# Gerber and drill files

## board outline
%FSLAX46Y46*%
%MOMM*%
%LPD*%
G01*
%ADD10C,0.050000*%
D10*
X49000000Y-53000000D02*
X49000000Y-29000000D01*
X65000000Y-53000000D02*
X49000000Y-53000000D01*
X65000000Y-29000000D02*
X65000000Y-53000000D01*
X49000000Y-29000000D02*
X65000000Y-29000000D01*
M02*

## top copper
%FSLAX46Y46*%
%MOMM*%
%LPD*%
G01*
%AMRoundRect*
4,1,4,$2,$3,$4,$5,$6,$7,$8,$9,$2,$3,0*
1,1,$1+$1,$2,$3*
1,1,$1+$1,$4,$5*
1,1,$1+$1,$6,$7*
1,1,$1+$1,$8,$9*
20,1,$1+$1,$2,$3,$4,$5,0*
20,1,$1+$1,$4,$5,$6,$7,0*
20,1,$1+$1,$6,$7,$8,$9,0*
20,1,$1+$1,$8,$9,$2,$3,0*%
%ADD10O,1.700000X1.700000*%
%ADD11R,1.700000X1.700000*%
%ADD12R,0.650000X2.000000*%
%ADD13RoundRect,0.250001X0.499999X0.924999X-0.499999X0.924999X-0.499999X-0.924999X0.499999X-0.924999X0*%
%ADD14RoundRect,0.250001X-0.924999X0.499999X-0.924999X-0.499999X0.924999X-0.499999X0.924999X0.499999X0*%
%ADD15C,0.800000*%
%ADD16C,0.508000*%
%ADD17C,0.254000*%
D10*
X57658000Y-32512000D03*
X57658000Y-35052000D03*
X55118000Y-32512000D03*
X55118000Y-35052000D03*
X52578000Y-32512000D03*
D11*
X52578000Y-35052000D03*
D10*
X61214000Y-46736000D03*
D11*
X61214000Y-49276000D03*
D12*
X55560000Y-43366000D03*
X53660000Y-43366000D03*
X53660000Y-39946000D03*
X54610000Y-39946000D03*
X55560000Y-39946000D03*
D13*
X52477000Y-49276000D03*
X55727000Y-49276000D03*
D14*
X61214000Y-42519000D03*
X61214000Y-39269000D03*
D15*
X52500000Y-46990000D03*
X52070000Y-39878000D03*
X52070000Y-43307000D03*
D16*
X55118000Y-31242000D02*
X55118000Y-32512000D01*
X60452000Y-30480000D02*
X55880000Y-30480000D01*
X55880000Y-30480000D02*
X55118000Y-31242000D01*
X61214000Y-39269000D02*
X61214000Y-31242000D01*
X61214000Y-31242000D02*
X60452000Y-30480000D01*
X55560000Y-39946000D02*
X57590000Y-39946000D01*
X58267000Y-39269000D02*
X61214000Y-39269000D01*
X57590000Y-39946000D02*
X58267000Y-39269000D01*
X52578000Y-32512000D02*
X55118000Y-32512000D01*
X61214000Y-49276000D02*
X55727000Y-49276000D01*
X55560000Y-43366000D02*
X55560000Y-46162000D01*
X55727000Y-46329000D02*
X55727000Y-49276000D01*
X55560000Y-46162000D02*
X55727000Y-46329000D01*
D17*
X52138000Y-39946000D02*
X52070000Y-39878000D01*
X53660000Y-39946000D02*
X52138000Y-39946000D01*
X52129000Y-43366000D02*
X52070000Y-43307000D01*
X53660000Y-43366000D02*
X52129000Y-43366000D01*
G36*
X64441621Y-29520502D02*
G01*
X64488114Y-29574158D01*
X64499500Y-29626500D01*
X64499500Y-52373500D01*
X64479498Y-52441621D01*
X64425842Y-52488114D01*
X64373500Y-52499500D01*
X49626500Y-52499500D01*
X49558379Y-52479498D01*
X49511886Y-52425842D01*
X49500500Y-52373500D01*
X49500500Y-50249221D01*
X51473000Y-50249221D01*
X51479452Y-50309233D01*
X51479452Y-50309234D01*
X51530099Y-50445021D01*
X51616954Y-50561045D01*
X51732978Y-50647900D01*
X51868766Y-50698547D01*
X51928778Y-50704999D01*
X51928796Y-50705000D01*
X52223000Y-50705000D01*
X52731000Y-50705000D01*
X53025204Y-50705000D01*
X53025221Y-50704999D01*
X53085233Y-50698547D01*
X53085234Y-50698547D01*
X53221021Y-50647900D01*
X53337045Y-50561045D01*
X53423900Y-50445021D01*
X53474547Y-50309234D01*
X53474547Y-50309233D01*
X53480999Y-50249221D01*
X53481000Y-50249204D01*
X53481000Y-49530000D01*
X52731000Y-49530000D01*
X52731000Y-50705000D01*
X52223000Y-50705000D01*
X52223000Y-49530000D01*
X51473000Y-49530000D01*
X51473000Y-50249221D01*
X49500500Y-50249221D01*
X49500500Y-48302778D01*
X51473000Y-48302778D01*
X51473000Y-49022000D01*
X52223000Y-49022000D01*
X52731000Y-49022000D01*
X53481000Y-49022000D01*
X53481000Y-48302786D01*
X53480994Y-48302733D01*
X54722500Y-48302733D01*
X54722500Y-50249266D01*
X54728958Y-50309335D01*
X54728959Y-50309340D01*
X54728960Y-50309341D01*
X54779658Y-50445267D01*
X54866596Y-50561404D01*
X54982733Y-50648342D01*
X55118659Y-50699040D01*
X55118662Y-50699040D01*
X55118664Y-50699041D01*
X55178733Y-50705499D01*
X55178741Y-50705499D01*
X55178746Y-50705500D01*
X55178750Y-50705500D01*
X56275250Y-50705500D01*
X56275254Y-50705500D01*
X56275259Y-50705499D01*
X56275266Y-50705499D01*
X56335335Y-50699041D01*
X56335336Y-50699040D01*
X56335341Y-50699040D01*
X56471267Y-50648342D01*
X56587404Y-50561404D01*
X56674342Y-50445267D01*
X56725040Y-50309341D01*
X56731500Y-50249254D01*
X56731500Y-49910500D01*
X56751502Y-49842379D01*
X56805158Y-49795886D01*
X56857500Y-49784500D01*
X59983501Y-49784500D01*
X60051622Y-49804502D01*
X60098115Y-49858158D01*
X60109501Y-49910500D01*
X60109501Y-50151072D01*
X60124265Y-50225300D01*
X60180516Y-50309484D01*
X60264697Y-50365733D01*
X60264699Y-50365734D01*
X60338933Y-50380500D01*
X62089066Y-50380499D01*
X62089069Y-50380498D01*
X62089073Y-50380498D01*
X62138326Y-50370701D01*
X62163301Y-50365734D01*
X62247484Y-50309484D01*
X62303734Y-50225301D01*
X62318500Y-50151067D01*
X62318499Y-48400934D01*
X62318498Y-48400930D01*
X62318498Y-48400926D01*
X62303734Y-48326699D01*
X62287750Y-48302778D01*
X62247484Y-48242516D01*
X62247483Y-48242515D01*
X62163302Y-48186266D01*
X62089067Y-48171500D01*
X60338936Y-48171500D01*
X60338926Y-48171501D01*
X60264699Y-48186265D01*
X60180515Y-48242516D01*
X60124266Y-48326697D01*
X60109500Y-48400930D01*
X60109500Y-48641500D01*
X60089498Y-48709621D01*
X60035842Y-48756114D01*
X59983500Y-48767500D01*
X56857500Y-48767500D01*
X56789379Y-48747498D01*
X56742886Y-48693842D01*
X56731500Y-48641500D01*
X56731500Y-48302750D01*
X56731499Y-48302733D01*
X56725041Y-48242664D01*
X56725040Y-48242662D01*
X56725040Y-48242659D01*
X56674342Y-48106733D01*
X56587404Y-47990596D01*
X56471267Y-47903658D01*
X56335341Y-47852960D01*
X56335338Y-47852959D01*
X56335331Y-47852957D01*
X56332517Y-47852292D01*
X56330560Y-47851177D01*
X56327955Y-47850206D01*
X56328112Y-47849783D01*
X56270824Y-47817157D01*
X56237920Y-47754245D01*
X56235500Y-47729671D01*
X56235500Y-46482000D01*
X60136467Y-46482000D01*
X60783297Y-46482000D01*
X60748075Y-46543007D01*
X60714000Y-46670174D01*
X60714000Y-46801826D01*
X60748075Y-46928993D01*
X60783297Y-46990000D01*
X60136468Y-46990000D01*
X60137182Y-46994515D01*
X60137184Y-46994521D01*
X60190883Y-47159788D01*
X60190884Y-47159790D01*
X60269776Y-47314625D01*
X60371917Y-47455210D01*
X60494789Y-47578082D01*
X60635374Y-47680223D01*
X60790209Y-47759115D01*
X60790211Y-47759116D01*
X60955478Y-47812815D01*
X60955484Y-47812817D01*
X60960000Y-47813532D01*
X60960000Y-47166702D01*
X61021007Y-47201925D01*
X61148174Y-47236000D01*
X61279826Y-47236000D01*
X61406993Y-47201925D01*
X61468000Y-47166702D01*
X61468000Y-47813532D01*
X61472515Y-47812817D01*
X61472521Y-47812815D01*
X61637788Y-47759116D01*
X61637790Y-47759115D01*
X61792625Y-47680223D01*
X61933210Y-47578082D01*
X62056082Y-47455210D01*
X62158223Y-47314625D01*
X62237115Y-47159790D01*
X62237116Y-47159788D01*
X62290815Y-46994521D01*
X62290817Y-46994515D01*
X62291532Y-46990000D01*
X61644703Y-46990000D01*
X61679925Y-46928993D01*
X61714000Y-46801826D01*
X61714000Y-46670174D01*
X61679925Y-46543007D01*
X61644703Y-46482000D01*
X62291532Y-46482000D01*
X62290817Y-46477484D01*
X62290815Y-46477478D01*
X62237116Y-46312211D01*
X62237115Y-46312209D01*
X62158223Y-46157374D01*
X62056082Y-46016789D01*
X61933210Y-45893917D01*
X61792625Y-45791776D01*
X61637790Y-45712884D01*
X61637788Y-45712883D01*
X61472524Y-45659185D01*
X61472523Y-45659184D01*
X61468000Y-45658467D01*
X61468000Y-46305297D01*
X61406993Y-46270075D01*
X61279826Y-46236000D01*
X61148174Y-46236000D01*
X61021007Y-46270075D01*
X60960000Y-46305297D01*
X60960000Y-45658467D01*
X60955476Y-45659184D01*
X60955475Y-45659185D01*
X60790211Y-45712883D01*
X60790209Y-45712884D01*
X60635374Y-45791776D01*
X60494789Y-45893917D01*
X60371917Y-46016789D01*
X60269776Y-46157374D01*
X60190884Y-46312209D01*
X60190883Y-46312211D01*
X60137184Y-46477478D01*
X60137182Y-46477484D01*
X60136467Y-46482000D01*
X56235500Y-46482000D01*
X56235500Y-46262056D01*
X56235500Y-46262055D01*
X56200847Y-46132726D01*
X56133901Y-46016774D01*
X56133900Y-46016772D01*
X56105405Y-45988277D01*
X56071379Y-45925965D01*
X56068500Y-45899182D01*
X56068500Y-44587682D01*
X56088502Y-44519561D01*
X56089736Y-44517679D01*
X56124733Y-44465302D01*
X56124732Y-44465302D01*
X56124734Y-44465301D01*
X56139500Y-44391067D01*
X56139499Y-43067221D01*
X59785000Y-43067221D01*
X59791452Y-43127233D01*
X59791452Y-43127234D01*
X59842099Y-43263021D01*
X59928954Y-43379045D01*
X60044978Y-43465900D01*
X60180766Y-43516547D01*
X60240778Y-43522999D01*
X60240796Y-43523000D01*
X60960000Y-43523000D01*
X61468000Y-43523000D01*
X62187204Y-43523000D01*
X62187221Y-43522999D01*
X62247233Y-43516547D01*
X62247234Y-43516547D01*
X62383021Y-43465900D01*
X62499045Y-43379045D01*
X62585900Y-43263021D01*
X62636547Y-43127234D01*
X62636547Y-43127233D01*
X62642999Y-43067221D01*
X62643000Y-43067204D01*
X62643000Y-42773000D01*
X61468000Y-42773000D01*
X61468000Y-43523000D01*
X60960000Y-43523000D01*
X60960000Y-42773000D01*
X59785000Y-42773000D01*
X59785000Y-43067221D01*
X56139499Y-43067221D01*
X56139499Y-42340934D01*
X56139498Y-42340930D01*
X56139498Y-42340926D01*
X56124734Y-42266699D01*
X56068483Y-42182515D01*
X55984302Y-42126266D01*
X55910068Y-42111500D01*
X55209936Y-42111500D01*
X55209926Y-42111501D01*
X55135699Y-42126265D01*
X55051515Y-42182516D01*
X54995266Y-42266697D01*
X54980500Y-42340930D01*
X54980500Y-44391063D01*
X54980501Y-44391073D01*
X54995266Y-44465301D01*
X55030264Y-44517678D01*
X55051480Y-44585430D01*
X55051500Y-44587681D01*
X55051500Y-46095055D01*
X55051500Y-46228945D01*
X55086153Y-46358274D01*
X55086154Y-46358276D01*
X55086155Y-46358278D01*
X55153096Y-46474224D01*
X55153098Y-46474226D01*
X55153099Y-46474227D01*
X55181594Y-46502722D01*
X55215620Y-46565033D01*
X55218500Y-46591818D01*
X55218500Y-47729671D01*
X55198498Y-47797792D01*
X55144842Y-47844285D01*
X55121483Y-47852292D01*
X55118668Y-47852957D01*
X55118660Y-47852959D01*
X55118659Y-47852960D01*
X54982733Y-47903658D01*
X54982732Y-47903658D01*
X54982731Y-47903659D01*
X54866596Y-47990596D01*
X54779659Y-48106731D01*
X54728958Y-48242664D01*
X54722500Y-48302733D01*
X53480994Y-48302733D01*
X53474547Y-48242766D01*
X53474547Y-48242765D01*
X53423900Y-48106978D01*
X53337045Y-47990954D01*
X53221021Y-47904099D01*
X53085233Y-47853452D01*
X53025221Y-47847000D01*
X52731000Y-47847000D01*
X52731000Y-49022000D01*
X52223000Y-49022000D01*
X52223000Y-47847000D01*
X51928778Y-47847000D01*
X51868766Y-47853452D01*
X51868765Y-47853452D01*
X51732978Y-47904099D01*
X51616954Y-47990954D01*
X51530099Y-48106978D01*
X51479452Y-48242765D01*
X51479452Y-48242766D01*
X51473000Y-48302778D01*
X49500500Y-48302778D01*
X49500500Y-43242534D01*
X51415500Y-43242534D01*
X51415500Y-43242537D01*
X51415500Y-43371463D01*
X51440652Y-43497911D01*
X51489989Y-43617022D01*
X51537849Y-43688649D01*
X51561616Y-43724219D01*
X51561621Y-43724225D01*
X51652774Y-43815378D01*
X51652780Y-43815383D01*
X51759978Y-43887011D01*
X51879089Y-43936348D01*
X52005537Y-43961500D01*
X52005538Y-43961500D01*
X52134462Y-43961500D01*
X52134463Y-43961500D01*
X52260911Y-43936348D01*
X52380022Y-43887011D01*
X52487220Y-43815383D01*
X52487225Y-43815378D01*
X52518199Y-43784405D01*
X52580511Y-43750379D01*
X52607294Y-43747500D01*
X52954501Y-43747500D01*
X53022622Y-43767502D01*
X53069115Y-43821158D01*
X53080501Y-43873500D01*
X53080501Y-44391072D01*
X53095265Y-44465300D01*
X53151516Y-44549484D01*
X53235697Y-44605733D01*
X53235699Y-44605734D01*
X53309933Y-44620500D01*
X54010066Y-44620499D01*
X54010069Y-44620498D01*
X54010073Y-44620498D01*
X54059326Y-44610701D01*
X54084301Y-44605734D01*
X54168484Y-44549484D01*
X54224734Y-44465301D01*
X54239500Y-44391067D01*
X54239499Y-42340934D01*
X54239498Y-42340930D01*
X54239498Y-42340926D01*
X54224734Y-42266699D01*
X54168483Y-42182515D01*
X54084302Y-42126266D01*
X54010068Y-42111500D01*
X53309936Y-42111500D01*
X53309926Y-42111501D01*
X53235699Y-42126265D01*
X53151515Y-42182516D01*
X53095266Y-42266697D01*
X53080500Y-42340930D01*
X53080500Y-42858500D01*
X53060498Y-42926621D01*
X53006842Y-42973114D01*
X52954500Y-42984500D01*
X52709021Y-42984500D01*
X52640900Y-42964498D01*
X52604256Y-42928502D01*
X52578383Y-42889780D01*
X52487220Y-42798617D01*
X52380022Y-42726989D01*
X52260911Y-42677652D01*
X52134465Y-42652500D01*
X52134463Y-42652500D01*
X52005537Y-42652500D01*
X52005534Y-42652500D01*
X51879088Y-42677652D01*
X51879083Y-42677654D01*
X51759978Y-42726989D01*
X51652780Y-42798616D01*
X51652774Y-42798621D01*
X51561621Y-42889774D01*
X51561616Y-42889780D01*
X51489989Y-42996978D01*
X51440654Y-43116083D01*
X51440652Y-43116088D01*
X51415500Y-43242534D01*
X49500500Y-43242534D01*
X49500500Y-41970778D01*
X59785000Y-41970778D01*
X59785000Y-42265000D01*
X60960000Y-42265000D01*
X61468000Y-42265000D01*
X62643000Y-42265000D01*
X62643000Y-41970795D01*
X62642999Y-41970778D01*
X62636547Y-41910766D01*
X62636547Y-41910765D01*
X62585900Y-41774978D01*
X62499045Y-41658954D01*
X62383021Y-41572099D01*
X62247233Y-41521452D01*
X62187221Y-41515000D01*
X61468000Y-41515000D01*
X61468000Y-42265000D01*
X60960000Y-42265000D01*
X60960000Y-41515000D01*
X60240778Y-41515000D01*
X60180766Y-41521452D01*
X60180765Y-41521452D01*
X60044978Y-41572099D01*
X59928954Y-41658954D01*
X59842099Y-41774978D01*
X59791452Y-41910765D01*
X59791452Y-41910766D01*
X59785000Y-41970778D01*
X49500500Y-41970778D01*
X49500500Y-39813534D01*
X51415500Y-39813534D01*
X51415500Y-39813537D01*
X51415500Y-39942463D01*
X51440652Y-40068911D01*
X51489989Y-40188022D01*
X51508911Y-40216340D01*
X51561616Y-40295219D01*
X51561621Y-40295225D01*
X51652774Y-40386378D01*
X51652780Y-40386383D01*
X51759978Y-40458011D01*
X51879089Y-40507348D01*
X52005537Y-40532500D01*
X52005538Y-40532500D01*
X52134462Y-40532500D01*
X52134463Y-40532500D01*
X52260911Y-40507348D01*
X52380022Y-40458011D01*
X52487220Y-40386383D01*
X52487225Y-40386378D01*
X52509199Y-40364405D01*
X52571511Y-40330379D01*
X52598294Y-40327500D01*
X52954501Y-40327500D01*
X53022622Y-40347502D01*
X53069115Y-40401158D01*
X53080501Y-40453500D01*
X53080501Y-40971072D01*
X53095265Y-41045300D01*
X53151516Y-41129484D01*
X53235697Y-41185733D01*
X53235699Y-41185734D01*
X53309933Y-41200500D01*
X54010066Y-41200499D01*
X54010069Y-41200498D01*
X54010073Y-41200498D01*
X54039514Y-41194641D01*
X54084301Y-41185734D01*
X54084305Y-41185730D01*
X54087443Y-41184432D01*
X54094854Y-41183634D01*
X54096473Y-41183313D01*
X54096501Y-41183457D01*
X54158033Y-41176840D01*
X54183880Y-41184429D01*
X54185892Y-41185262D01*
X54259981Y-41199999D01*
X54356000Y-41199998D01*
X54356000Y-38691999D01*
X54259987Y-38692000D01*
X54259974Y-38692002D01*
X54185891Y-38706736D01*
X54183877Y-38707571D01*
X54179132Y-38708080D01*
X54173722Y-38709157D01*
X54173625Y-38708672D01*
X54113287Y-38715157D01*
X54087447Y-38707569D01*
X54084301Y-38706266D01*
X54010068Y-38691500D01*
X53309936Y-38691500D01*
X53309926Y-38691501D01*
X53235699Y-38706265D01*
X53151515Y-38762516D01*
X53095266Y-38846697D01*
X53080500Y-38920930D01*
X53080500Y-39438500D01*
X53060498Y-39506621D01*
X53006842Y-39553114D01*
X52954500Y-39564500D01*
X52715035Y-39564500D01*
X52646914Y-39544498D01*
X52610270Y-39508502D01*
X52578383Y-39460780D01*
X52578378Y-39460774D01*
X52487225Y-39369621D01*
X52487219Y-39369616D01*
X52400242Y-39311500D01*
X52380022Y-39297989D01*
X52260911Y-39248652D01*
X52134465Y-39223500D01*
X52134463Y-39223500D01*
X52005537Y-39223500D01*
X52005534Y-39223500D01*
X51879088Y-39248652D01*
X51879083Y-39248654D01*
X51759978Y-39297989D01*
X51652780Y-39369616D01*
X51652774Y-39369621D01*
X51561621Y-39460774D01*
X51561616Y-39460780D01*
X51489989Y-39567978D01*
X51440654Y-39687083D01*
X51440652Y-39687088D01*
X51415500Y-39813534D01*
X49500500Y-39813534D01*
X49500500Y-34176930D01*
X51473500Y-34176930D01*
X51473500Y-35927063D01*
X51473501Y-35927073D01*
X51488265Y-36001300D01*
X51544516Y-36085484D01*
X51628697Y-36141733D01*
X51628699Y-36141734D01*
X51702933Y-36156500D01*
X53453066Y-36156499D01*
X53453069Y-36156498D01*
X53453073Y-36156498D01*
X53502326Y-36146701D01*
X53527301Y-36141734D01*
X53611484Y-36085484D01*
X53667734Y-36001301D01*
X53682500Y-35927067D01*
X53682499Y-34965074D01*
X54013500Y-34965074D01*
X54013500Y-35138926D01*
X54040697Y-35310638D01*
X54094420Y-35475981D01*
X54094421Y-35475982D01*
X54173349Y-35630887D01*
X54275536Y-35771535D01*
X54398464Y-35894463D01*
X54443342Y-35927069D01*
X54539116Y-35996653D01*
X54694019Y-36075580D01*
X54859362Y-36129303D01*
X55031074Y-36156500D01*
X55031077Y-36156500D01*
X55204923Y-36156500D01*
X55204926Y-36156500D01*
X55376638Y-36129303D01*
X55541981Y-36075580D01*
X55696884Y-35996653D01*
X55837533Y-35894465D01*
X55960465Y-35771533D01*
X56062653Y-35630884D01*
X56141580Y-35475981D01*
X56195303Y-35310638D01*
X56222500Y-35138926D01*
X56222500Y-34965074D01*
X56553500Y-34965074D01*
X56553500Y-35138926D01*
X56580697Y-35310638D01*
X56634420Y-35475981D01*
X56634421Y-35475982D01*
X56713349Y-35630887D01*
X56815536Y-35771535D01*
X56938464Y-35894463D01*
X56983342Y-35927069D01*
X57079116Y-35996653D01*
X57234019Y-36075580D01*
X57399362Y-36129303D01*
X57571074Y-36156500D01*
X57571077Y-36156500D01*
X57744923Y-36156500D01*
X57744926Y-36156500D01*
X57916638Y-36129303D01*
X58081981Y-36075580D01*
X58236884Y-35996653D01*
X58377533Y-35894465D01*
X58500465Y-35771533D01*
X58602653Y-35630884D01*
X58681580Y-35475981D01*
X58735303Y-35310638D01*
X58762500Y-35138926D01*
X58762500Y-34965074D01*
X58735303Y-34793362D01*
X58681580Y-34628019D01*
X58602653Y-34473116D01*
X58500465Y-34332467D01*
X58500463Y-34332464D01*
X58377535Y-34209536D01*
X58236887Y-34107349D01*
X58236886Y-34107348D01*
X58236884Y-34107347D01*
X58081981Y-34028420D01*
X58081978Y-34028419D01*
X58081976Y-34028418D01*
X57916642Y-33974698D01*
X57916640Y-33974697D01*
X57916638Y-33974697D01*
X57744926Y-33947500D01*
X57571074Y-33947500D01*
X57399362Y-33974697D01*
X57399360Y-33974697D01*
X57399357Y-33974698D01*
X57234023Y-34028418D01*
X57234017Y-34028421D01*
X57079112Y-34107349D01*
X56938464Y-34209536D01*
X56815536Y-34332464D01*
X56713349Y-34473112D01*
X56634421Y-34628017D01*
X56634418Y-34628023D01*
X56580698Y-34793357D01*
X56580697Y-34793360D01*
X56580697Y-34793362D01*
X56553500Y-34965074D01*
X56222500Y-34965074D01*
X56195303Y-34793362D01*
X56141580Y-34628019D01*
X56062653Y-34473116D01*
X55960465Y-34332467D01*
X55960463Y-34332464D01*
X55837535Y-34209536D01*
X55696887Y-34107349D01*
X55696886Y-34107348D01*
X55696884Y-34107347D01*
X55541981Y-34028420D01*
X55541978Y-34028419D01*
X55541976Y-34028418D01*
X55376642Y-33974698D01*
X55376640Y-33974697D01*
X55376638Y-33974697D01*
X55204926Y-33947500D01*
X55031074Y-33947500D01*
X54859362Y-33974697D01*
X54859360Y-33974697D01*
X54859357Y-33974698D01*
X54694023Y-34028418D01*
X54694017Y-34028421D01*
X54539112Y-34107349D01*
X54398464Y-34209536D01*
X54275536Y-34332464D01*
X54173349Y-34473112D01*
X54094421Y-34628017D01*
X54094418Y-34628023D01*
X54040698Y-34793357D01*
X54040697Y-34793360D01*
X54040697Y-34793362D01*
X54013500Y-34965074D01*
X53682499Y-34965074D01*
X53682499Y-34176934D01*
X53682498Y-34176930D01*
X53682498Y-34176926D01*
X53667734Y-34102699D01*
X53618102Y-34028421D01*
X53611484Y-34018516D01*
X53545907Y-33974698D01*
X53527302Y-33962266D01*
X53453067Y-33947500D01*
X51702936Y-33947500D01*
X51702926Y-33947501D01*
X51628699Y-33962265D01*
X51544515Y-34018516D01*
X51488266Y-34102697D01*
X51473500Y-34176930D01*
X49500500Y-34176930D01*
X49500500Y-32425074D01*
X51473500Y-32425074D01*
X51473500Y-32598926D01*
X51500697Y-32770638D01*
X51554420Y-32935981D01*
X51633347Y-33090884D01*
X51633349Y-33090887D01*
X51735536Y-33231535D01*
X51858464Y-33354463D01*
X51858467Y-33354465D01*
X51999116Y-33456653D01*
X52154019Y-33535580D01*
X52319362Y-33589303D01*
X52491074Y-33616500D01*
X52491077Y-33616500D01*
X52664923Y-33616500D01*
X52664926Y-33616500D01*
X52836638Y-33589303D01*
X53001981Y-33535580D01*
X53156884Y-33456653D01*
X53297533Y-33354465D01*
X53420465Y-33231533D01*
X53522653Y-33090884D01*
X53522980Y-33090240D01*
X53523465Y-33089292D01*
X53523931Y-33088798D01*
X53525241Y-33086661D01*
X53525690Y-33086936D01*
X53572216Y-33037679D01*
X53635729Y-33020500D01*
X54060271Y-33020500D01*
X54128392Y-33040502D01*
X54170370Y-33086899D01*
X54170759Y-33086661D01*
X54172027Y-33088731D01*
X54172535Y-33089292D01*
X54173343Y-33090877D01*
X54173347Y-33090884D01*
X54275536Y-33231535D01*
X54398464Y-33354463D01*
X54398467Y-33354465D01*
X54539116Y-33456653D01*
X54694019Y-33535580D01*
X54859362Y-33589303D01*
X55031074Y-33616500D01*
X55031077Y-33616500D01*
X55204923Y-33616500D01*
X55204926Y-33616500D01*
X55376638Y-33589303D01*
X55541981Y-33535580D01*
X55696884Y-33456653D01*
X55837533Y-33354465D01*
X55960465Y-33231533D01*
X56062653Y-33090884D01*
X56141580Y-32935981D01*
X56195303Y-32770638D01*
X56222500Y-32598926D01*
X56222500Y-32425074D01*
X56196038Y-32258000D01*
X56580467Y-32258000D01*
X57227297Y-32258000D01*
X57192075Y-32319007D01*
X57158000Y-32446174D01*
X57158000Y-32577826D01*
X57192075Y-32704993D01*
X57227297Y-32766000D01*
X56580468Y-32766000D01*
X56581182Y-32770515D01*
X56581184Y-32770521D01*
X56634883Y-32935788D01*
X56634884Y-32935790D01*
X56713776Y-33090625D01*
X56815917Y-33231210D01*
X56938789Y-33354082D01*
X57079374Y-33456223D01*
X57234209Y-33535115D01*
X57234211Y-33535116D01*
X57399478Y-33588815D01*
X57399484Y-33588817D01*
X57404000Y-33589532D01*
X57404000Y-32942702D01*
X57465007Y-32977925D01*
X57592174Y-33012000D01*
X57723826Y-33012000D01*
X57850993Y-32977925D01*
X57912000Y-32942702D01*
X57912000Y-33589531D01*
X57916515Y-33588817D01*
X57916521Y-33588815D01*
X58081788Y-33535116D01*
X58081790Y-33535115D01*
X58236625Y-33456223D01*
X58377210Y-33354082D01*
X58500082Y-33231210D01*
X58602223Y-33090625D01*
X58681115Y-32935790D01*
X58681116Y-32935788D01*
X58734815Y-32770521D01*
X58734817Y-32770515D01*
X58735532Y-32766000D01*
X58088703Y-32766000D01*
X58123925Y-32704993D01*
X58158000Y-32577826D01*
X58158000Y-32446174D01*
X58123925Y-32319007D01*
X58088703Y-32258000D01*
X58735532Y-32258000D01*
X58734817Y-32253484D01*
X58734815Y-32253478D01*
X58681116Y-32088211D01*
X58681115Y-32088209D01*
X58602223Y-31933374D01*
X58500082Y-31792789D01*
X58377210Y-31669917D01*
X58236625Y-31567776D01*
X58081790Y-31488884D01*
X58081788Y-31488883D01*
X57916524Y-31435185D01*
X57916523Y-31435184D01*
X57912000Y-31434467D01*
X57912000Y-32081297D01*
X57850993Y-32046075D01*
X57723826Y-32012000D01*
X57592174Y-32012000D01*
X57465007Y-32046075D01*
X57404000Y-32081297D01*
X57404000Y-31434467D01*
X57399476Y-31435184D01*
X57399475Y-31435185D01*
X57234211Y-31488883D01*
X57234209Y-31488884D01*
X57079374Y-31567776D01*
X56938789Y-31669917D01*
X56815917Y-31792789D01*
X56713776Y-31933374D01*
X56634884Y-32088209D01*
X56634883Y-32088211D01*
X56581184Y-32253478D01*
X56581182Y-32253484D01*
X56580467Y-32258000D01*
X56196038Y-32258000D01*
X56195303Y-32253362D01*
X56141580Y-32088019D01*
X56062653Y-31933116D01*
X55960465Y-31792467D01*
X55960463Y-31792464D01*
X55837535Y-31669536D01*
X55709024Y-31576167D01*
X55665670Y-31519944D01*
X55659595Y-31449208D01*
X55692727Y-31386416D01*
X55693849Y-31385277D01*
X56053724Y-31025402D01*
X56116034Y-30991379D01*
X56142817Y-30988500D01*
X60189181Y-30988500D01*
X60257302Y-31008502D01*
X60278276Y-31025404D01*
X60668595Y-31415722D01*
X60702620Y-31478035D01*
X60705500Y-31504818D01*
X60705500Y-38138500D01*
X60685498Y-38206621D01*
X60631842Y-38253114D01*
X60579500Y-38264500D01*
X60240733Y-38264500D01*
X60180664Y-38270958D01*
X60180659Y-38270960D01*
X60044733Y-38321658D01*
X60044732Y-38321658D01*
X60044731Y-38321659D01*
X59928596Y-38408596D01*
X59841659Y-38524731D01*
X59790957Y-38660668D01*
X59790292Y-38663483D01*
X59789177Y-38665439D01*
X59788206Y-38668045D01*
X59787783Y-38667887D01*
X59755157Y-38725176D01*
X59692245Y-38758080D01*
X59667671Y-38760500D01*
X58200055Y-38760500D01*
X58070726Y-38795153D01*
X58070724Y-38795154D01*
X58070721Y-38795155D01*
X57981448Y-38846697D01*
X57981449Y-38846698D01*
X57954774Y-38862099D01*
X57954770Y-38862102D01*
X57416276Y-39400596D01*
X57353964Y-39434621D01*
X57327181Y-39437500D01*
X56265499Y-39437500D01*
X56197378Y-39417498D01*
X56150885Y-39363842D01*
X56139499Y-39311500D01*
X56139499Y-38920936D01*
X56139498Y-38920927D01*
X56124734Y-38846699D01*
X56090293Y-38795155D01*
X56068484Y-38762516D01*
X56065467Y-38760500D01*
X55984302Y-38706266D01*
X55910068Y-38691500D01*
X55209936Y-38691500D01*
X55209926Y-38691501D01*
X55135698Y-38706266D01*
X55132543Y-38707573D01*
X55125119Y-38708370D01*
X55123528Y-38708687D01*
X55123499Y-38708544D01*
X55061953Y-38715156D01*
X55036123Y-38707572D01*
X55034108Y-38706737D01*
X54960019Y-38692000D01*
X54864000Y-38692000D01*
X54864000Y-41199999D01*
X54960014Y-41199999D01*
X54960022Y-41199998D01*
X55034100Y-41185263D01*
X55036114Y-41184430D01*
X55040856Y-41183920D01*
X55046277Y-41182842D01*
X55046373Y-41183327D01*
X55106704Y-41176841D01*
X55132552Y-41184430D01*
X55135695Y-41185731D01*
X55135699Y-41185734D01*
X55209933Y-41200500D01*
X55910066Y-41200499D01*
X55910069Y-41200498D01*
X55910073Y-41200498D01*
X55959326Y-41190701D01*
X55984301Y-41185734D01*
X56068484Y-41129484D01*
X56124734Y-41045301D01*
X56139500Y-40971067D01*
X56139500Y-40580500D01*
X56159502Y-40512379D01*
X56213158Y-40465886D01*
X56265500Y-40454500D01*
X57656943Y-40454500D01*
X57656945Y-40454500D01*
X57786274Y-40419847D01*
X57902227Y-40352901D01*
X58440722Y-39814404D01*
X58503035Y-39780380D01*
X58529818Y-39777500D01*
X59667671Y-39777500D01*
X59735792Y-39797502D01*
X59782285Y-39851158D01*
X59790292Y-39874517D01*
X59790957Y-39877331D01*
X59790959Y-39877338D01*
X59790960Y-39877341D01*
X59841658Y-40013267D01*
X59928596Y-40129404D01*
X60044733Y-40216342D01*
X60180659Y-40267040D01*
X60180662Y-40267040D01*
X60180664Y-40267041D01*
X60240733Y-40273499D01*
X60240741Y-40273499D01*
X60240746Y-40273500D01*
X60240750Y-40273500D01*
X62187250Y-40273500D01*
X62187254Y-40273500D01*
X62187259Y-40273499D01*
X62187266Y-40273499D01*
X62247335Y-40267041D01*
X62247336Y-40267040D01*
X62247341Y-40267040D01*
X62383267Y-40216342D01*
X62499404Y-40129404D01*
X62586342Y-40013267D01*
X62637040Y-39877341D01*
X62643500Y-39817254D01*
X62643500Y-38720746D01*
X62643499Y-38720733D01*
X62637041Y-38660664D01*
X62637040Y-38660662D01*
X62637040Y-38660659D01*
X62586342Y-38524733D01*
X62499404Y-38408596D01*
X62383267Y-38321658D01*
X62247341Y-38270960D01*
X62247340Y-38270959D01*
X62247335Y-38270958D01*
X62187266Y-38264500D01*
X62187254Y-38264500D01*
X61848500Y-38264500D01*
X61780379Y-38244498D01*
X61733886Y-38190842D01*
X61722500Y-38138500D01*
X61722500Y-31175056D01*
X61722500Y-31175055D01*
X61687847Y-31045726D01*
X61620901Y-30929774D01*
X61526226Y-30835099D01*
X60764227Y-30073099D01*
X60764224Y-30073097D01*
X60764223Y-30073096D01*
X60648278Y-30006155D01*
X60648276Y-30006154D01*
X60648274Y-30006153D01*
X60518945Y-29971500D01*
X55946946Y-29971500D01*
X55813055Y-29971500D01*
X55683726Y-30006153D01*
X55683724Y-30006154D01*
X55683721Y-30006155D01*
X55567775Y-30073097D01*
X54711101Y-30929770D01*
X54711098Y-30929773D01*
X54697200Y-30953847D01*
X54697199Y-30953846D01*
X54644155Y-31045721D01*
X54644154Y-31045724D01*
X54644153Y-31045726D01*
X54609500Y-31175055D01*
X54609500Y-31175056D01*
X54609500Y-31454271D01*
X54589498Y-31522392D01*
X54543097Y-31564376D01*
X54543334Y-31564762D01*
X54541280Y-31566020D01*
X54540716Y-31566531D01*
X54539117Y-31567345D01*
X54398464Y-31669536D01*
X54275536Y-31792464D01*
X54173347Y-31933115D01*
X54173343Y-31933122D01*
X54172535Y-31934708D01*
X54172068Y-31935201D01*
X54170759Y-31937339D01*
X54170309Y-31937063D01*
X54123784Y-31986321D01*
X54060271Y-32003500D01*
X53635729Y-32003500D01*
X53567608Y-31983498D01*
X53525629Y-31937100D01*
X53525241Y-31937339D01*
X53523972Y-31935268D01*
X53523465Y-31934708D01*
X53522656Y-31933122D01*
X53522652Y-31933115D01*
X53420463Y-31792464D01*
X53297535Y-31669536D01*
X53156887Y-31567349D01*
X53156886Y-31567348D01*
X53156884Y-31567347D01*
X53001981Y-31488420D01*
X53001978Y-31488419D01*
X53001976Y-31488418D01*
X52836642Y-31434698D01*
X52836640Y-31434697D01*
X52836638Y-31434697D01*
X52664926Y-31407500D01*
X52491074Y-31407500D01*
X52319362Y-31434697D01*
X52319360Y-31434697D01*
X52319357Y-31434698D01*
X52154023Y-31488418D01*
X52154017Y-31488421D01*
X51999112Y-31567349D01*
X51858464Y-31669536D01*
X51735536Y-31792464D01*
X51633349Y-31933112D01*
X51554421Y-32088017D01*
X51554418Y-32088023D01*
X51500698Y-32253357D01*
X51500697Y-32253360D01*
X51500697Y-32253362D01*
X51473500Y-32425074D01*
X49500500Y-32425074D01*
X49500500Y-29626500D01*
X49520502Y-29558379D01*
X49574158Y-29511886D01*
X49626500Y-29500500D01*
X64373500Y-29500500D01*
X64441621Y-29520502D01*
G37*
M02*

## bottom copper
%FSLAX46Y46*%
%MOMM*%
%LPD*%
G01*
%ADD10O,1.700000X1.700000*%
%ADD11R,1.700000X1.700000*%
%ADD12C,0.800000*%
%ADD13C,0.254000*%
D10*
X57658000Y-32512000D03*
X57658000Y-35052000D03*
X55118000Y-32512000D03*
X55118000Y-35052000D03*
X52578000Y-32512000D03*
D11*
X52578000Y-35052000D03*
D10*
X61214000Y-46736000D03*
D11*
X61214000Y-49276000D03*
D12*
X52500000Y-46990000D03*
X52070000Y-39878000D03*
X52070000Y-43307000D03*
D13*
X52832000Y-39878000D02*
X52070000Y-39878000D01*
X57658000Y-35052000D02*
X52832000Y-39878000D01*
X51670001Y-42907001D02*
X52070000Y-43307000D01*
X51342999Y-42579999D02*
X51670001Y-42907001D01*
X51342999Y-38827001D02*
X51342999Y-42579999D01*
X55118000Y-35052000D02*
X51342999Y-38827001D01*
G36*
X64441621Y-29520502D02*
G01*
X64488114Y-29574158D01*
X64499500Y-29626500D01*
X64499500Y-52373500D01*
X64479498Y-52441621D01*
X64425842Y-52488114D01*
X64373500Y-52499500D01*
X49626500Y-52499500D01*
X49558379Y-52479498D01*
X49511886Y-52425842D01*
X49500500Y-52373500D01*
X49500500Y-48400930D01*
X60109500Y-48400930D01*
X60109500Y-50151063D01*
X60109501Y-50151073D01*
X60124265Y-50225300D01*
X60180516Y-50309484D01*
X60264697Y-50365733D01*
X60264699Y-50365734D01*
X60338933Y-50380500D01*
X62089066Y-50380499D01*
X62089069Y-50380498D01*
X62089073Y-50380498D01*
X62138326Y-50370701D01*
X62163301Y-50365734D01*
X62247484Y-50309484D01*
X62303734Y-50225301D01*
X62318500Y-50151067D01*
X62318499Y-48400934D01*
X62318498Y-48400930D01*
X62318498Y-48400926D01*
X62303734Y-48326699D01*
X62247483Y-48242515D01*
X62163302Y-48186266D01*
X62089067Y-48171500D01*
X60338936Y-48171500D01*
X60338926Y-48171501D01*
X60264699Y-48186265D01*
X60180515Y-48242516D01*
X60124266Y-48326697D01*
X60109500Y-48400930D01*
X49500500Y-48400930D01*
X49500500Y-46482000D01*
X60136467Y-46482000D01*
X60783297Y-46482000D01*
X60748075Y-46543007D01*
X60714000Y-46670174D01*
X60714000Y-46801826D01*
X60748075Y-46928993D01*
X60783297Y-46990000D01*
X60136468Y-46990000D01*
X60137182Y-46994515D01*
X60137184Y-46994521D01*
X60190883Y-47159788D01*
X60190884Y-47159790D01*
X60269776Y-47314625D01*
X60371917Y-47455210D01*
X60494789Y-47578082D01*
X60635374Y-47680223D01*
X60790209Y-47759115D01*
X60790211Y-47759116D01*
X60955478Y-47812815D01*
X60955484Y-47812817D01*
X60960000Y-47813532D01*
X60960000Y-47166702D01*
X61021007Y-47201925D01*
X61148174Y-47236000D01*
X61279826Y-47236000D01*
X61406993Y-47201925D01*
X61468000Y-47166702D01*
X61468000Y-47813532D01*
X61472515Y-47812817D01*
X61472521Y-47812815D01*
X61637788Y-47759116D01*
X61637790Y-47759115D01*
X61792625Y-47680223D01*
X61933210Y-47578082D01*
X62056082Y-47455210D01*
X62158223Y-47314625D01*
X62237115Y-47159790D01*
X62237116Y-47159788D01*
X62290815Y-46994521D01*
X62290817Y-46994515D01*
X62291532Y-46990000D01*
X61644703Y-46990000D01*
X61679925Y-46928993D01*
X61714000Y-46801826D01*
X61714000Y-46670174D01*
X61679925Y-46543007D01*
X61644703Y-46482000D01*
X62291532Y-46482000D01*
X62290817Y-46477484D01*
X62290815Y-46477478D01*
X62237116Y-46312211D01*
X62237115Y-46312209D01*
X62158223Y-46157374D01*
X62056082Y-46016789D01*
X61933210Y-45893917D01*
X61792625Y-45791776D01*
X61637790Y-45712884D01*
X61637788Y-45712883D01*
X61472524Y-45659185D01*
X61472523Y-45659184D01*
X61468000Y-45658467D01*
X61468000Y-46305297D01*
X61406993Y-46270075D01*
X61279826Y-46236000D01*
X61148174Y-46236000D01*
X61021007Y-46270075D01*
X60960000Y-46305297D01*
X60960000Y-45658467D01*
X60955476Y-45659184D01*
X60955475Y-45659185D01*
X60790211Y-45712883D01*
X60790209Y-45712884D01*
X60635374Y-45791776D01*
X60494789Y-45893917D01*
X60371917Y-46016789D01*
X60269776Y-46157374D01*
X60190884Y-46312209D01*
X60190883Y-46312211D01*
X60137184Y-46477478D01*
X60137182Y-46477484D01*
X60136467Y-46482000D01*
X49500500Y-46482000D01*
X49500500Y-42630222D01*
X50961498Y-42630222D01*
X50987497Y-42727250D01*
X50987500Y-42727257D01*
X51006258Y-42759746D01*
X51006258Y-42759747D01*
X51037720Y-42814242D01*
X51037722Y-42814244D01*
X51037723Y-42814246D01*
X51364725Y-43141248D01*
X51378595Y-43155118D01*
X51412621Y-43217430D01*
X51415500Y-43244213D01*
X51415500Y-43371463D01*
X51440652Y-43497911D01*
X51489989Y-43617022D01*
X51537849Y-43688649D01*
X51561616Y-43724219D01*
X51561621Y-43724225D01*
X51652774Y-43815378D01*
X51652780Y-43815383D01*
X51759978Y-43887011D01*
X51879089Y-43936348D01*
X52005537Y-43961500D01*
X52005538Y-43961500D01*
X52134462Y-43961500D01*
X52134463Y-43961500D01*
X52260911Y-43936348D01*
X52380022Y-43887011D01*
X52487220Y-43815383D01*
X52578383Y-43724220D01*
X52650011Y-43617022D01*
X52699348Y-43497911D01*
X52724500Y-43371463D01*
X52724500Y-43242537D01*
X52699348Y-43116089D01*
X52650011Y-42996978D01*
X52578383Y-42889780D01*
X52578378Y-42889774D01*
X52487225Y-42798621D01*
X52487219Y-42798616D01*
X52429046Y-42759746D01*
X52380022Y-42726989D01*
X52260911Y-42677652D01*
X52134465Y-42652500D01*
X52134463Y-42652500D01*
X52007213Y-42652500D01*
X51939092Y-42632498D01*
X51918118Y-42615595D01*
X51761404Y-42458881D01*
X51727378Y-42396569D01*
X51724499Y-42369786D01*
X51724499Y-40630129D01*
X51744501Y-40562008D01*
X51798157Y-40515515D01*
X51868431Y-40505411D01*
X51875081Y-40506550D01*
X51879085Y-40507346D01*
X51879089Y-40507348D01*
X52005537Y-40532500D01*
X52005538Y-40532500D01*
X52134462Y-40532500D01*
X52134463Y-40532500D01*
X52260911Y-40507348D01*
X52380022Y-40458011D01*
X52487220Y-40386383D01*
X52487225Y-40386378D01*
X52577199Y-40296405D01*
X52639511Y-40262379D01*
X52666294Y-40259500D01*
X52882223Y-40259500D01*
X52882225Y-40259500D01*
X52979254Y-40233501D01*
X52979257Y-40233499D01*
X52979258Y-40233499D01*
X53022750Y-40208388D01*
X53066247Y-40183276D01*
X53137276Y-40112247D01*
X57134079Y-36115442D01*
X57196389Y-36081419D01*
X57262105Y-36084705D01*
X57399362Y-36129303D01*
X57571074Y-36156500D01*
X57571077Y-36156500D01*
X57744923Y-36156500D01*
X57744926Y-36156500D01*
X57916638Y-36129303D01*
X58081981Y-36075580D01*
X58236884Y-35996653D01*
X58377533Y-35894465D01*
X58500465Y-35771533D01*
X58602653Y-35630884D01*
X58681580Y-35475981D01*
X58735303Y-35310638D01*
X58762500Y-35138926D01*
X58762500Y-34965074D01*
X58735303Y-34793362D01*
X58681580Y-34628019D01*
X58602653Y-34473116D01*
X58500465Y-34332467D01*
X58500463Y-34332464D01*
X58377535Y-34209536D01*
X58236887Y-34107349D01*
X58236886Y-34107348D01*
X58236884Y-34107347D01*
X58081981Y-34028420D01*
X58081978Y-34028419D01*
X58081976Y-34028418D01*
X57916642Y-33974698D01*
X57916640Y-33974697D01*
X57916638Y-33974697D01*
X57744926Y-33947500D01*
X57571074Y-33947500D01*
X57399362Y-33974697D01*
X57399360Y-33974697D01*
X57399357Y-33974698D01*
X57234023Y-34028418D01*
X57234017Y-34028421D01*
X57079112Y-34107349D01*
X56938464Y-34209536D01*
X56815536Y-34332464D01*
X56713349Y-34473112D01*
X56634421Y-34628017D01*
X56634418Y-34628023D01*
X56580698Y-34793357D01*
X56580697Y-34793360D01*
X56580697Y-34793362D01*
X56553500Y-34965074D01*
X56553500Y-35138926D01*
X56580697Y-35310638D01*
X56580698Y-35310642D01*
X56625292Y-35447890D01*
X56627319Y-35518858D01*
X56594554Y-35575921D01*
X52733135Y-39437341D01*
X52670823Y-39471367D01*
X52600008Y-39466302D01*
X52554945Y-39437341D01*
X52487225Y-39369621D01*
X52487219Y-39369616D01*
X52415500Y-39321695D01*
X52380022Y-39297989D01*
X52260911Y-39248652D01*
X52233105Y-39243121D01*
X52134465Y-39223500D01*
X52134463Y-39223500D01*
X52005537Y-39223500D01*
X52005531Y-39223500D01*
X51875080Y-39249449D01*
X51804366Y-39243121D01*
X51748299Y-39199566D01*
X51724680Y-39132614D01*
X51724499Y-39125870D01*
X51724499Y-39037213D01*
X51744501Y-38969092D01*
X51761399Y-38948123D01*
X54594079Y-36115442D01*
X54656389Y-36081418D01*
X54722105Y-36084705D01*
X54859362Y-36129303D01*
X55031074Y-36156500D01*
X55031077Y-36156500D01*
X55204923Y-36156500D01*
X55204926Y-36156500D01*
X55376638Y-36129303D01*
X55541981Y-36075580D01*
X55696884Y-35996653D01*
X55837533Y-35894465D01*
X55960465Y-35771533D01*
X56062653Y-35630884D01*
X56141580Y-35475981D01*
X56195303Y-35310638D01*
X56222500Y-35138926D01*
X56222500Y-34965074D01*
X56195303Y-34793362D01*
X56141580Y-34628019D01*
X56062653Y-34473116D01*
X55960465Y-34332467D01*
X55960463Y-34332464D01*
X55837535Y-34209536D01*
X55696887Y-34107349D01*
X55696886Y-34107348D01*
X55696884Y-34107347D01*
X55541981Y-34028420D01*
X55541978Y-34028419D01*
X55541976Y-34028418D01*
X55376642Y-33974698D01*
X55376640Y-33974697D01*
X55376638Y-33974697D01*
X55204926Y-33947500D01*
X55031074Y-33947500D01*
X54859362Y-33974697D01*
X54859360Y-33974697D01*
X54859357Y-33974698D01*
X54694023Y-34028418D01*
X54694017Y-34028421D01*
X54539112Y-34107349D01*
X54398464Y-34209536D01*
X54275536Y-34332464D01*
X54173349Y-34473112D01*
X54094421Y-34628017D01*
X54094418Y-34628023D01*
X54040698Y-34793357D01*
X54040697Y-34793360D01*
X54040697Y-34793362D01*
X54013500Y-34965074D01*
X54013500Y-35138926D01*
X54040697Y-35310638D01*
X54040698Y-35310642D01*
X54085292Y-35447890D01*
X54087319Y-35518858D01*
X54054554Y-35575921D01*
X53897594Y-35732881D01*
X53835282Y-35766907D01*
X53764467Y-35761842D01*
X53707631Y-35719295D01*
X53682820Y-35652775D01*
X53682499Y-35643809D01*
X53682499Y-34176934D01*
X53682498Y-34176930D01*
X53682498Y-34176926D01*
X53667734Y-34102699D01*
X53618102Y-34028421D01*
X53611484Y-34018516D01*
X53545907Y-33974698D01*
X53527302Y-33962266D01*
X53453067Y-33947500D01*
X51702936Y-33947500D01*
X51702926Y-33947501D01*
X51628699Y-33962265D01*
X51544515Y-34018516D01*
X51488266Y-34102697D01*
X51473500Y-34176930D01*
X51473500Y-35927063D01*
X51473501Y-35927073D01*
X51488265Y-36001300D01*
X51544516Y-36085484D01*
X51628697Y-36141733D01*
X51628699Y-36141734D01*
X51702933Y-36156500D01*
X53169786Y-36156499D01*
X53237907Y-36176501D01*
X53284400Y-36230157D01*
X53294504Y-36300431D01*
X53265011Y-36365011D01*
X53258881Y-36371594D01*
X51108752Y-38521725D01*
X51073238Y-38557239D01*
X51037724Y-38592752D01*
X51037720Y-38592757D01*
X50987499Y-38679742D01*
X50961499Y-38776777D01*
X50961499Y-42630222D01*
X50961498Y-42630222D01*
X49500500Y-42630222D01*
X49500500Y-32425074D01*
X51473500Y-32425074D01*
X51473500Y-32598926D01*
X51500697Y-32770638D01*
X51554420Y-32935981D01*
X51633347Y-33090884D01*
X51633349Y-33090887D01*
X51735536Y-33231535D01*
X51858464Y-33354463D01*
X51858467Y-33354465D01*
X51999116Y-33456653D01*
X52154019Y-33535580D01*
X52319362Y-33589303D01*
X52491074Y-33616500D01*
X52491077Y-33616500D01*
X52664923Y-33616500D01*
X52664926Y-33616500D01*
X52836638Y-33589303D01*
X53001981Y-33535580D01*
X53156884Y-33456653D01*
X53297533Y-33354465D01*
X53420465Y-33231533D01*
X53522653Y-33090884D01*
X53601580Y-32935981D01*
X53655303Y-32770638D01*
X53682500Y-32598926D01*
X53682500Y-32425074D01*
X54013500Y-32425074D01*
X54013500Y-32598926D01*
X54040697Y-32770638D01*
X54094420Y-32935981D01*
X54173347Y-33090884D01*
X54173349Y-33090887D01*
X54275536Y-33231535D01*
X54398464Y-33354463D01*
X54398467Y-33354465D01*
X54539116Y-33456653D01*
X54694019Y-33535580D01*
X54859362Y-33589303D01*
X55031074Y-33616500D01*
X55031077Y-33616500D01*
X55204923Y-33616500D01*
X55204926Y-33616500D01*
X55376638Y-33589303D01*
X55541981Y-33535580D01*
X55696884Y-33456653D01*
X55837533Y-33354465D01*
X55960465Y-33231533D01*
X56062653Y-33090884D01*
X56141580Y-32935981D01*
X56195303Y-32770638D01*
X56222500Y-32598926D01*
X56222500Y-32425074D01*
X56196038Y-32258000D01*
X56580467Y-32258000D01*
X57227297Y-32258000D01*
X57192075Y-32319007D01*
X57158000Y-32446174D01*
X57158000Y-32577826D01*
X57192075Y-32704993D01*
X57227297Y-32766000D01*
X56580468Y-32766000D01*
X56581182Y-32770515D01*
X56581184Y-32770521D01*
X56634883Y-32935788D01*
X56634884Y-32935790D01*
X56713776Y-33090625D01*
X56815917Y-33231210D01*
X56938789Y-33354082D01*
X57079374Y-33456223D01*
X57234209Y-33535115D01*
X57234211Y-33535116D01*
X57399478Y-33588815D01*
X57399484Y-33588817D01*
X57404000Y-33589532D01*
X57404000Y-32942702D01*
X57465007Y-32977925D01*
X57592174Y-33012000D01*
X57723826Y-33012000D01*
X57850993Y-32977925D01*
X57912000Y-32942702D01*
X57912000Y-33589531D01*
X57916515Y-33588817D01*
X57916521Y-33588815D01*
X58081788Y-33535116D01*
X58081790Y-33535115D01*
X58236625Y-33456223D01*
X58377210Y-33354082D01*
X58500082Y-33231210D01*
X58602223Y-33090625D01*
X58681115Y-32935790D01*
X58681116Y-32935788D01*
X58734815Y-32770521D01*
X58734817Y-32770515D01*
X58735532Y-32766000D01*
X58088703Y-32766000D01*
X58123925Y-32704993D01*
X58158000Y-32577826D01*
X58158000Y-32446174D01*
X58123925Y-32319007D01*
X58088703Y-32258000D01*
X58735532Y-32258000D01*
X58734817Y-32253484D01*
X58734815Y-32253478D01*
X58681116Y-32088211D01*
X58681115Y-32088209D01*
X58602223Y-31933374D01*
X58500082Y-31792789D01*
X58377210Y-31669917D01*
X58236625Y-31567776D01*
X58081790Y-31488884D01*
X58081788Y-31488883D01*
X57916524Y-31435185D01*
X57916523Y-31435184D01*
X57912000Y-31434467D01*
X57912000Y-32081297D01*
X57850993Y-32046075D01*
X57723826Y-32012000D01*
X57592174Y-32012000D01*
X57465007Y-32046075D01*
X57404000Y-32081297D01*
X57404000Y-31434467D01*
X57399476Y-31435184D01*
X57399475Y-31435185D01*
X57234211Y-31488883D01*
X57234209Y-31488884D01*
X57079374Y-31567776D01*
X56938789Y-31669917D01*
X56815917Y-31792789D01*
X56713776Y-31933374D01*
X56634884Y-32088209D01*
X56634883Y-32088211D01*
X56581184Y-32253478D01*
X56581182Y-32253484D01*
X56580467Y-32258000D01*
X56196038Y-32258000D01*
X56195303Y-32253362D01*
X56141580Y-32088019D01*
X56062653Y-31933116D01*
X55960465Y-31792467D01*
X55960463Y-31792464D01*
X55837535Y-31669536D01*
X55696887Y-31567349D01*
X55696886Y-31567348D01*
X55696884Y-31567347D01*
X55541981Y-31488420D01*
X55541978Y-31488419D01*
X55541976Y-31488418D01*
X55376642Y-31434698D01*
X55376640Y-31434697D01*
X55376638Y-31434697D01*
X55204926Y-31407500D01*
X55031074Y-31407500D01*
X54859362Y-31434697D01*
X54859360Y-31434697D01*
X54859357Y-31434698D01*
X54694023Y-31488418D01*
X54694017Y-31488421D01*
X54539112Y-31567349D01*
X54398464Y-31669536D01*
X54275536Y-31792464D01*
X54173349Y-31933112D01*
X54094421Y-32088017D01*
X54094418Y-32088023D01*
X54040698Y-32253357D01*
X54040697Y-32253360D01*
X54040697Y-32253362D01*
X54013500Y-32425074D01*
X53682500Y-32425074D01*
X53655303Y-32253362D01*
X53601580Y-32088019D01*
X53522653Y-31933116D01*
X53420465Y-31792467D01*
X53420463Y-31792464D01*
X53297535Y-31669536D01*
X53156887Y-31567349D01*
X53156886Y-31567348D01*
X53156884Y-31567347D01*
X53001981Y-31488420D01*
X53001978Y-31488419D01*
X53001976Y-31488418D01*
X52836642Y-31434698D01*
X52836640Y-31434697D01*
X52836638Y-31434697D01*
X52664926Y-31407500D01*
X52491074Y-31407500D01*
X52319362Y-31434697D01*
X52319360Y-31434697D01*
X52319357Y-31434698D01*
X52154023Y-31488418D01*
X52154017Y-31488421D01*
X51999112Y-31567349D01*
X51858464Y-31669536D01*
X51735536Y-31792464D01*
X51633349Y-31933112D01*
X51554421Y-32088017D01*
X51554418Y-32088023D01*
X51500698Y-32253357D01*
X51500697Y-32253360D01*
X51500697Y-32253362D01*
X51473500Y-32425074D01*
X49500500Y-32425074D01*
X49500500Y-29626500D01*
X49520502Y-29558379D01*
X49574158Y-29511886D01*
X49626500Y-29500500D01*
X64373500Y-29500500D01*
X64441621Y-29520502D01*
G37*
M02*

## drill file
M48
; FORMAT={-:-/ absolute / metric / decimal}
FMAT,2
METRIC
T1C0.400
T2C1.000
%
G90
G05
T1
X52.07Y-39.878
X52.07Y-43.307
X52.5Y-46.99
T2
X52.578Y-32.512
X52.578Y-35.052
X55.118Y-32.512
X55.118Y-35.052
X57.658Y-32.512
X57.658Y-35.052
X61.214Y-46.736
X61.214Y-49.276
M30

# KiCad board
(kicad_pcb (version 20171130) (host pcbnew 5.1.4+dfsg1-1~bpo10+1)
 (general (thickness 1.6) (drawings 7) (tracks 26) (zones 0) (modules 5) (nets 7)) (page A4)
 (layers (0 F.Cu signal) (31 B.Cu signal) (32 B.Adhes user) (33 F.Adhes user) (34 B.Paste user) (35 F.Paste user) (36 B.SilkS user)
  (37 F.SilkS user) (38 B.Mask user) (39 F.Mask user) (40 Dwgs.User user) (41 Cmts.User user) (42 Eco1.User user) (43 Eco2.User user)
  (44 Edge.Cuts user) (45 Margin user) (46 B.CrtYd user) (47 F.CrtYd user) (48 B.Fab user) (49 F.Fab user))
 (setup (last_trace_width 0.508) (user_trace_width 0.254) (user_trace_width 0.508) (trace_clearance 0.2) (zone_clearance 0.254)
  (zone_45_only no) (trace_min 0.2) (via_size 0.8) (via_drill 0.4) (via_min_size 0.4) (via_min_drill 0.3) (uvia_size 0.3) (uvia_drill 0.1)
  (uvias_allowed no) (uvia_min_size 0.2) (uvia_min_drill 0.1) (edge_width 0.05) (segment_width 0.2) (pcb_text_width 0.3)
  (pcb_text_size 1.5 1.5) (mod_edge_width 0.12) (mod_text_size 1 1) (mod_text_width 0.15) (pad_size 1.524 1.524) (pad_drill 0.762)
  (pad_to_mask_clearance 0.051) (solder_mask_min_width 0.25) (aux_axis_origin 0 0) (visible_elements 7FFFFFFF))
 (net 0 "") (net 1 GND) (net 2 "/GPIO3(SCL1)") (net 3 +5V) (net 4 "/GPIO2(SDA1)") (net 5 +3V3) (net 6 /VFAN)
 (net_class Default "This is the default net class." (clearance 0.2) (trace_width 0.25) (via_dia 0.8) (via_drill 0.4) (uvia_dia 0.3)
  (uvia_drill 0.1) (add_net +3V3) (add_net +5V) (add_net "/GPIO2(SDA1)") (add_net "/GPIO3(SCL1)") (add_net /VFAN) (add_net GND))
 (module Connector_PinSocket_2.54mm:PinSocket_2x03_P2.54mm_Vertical (layer B.Cu) (at 52.578 35.052 270)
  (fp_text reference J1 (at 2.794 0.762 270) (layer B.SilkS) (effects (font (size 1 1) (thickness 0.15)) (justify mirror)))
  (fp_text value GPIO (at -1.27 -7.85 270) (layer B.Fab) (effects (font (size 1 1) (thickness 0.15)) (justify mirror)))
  (pad 6 thru_hole oval (at -2.54 -5.08 270) (size 1.7 1.7) (drill 1) (layers *.Cu *.Mask) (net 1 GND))
  (pad 5 thru_hole oval (at 0 -5.08 270) (size 1.7 1.7) (drill 1) (layers *.Cu *.Mask) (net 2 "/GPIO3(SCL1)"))
  (pad 4 thru_hole oval (at -2.54 -2.54 270) (size 1.7 1.7) (drill 1) (layers *.Cu *.Mask) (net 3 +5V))
  (pad 3 thru_hole oval (at 0 -2.54 270) (size 1.7 1.7) (drill 1) (layers *.Cu *.Mask) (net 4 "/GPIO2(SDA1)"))
  (pad 2 thru_hole oval (at -2.54 0 270) (size 1.7 1.7) (drill 1) (layers *.Cu *.Mask) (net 3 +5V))
  (pad 1 thru_hole rect (at 0 0 270) (size 1.7 1.7) (drill 1) (layers *.Cu *.Mask) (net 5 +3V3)))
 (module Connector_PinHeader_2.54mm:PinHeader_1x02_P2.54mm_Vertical (layer F.Cu) (at 61.214 49.276 180)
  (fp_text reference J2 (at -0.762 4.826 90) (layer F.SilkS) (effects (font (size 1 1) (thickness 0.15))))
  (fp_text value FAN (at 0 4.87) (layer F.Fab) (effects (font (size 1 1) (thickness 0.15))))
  (pad 2 thru_hole oval (at 0 2.54 180) (size 1.7 1.7) (drill 1) (layers *.Cu *.Mask) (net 1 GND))
  (pad 1 thru_hole rect (at 0 0 180) (size 1.7 1.7) (drill 1) (layers *.Cu *.Mask) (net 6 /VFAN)))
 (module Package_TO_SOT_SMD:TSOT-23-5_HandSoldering (layer F.Cu) (at 54.61 41.656 270)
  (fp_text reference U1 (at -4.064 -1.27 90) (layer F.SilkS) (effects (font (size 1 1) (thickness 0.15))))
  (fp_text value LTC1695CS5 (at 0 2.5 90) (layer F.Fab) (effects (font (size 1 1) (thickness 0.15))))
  (pad 5 smd rect (at 1.71 -0.95 270) (size 2 0.65) (layers F.Cu F.Paste F.Mask) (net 6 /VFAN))
  (pad 4 smd rect (at 1.71 0.95 270) (size 2 0.65) (layers F.Cu F.Paste F.Mask) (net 4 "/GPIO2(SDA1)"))
  (pad 3 smd rect (at -1.71 0.95 270) (size 2 0.65) (layers F.Cu F.Paste F.Mask) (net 2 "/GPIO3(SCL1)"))
  (pad 2 smd rect (at -1.71 0 270) (size 2 0.65) (layers F.Cu F.Paste F.Mask) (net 1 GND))
  (pad 1 smd rect (at -1.71 -0.95 270) (size 2 0.65) (layers F.Cu F.Paste F.Mask) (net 3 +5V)))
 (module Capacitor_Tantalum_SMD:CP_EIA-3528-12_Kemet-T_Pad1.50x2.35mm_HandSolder (layer F.Cu) (at 54.102 49.276 180)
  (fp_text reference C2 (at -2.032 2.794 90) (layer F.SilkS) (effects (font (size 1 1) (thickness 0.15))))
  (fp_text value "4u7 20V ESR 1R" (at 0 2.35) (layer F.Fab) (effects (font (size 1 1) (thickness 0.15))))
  (pad 2 smd roundrect (at 1.625 0 180) (size 1.5 2.35) (layers F.Cu F.Paste F.Mask) (roundrect_rratio 0.166667) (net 1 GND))
  (pad 1 smd roundrect (at -1.625 0 180) (size 1.5 2.35) (layers F.Cu F.Paste F.Mask) (roundrect_rratio 0.166667) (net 6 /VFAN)))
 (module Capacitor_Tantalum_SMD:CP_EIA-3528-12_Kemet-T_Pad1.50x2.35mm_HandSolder (layer F.Cu) (at 61.214 40.894 270)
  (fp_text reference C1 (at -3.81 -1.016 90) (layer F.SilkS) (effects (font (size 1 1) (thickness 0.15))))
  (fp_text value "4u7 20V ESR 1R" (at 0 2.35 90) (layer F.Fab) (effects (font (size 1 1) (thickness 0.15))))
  (pad 2 smd roundrect (at 1.625 0 270) (size 1.5 2.35) (layers F.Cu F.Paste F.Mask) (roundrect_rratio 0.166667) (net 1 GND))
  (pad 1 smd roundrect (at -1.625 0 270) (size 1.5 2.35) (layers F.Cu F.Paste F.Mask) (roundrect_rratio 0.166667) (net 3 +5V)))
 (gr_line (start 49 53) (end 49 29) (layer Edge.Cuts) (width 0.05))
 (gr_line (start 65 53) (end 49 53) (layer Edge.Cuts) (width 0.05))
 (gr_line (start 65 29) (end 65 53) (layer Edge.Cuts) (width 0.05))
 (gr_line (start 49 29) (end 65 29) (layer Edge.Cuts) (width 0.05))
 (via (at 52.5 46.99) (size 0.8) (drill 0.4) (layers F.Cu B.Cu) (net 1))
 (segment (start 55.118 31.242) (end 55.118 32.512) (width 0.508) (layer F.Cu) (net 3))
 (segment (start 60.452 30.48) (end 55.88 30.48) (width 0.508) (layer F.Cu) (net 3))
 (segment (start 55.88 30.48) (end 55.118 31.242) (width 0.508) (layer F.Cu) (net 3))
 (segment (start 61.214 39.269) (end 61.214 31.242) (width 0.508) (layer F.Cu) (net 3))
 (segment (start 61.214 31.242) (end 60.452 30.48) (width 0.508) (layer F.Cu) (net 3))
 (segment (start 55.56 39.946) (end 57.59 39.946) (width 0.508) (layer F.Cu) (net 3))
 (segment (start 58.267 39.269) (end 61.214 39.269) (width 0.508) (layer F.Cu) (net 3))
 (segment (start 57.59 39.946) (end 58.267 39.269) (width 0.508) (layer F.Cu) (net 3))
 (segment (start 52.578 32.512) (end 55.118 32.512) (width 0.508) (layer F.Cu) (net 3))
 (segment (start 61.214 49.276) (end 55.727 49.276) (width 0.508) (layer F.Cu) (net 6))
 (segment (start 55.56 43.366) (end 55.56 46.162) (width 0.508) (layer F.Cu) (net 6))
 (segment (start 55.727 46.329) (end 55.727 49.276) (width 0.508) (layer F.Cu) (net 6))
 (segment (start 55.56 46.162) (end 55.727 46.329) (width 0.508) (layer F.Cu) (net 6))
 (via (at 52.07 39.878) (size 0.8) (drill 0.4) (layers F.Cu B.Cu) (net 2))
 (segment (start 52.138 39.946) (end 52.07 39.878) (width 0.254) (layer F.Cu) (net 2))
 (segment (start 53.66 39.946) (end 52.138 39.946) (width 0.254) (layer F.Cu) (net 2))
 (segment (start 52.832 39.878) (end 52.07 39.878) (width 0.254) (layer B.Cu) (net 2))
 (segment (start 57.658 35.052) (end 52.832 39.878) (width 0.254) (layer B.Cu) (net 2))
 (via (at 52.07 43.307) (size 0.8) (drill 0.4) (layers F.Cu B.Cu) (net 4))
 (segment (start 52.129 43.366) (end 52.07 43.307) (width 0.254) (layer F.Cu) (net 4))
 (segment (start 53.66 43.366) (end 52.129 43.366) (width 0.254) (layer F.Cu) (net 4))
 (segment (start 51.670001 42.907001) (end 52.07 43.307) (width 0.254) (layer B.Cu) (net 4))
 (segment (start 51.342999 42.579999) (end 51.670001 42.907001) (width 0.254) (layer B.Cu) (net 4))
 (segment (start 51.342999 38.827001) (end 51.342999 42.579999) (width 0.254) (layer B.Cu) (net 4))
 (segment (start 55.118 35.052) (end 51.342999 38.827001) (width 0.254) (layer B.Cu) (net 4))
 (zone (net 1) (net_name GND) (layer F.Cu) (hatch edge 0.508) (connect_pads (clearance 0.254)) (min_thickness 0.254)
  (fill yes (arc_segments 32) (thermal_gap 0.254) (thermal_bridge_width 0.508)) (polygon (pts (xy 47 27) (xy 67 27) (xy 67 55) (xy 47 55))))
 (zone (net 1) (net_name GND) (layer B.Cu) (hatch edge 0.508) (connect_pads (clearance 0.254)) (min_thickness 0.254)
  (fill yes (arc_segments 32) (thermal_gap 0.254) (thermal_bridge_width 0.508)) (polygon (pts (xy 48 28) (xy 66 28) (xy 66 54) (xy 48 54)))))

